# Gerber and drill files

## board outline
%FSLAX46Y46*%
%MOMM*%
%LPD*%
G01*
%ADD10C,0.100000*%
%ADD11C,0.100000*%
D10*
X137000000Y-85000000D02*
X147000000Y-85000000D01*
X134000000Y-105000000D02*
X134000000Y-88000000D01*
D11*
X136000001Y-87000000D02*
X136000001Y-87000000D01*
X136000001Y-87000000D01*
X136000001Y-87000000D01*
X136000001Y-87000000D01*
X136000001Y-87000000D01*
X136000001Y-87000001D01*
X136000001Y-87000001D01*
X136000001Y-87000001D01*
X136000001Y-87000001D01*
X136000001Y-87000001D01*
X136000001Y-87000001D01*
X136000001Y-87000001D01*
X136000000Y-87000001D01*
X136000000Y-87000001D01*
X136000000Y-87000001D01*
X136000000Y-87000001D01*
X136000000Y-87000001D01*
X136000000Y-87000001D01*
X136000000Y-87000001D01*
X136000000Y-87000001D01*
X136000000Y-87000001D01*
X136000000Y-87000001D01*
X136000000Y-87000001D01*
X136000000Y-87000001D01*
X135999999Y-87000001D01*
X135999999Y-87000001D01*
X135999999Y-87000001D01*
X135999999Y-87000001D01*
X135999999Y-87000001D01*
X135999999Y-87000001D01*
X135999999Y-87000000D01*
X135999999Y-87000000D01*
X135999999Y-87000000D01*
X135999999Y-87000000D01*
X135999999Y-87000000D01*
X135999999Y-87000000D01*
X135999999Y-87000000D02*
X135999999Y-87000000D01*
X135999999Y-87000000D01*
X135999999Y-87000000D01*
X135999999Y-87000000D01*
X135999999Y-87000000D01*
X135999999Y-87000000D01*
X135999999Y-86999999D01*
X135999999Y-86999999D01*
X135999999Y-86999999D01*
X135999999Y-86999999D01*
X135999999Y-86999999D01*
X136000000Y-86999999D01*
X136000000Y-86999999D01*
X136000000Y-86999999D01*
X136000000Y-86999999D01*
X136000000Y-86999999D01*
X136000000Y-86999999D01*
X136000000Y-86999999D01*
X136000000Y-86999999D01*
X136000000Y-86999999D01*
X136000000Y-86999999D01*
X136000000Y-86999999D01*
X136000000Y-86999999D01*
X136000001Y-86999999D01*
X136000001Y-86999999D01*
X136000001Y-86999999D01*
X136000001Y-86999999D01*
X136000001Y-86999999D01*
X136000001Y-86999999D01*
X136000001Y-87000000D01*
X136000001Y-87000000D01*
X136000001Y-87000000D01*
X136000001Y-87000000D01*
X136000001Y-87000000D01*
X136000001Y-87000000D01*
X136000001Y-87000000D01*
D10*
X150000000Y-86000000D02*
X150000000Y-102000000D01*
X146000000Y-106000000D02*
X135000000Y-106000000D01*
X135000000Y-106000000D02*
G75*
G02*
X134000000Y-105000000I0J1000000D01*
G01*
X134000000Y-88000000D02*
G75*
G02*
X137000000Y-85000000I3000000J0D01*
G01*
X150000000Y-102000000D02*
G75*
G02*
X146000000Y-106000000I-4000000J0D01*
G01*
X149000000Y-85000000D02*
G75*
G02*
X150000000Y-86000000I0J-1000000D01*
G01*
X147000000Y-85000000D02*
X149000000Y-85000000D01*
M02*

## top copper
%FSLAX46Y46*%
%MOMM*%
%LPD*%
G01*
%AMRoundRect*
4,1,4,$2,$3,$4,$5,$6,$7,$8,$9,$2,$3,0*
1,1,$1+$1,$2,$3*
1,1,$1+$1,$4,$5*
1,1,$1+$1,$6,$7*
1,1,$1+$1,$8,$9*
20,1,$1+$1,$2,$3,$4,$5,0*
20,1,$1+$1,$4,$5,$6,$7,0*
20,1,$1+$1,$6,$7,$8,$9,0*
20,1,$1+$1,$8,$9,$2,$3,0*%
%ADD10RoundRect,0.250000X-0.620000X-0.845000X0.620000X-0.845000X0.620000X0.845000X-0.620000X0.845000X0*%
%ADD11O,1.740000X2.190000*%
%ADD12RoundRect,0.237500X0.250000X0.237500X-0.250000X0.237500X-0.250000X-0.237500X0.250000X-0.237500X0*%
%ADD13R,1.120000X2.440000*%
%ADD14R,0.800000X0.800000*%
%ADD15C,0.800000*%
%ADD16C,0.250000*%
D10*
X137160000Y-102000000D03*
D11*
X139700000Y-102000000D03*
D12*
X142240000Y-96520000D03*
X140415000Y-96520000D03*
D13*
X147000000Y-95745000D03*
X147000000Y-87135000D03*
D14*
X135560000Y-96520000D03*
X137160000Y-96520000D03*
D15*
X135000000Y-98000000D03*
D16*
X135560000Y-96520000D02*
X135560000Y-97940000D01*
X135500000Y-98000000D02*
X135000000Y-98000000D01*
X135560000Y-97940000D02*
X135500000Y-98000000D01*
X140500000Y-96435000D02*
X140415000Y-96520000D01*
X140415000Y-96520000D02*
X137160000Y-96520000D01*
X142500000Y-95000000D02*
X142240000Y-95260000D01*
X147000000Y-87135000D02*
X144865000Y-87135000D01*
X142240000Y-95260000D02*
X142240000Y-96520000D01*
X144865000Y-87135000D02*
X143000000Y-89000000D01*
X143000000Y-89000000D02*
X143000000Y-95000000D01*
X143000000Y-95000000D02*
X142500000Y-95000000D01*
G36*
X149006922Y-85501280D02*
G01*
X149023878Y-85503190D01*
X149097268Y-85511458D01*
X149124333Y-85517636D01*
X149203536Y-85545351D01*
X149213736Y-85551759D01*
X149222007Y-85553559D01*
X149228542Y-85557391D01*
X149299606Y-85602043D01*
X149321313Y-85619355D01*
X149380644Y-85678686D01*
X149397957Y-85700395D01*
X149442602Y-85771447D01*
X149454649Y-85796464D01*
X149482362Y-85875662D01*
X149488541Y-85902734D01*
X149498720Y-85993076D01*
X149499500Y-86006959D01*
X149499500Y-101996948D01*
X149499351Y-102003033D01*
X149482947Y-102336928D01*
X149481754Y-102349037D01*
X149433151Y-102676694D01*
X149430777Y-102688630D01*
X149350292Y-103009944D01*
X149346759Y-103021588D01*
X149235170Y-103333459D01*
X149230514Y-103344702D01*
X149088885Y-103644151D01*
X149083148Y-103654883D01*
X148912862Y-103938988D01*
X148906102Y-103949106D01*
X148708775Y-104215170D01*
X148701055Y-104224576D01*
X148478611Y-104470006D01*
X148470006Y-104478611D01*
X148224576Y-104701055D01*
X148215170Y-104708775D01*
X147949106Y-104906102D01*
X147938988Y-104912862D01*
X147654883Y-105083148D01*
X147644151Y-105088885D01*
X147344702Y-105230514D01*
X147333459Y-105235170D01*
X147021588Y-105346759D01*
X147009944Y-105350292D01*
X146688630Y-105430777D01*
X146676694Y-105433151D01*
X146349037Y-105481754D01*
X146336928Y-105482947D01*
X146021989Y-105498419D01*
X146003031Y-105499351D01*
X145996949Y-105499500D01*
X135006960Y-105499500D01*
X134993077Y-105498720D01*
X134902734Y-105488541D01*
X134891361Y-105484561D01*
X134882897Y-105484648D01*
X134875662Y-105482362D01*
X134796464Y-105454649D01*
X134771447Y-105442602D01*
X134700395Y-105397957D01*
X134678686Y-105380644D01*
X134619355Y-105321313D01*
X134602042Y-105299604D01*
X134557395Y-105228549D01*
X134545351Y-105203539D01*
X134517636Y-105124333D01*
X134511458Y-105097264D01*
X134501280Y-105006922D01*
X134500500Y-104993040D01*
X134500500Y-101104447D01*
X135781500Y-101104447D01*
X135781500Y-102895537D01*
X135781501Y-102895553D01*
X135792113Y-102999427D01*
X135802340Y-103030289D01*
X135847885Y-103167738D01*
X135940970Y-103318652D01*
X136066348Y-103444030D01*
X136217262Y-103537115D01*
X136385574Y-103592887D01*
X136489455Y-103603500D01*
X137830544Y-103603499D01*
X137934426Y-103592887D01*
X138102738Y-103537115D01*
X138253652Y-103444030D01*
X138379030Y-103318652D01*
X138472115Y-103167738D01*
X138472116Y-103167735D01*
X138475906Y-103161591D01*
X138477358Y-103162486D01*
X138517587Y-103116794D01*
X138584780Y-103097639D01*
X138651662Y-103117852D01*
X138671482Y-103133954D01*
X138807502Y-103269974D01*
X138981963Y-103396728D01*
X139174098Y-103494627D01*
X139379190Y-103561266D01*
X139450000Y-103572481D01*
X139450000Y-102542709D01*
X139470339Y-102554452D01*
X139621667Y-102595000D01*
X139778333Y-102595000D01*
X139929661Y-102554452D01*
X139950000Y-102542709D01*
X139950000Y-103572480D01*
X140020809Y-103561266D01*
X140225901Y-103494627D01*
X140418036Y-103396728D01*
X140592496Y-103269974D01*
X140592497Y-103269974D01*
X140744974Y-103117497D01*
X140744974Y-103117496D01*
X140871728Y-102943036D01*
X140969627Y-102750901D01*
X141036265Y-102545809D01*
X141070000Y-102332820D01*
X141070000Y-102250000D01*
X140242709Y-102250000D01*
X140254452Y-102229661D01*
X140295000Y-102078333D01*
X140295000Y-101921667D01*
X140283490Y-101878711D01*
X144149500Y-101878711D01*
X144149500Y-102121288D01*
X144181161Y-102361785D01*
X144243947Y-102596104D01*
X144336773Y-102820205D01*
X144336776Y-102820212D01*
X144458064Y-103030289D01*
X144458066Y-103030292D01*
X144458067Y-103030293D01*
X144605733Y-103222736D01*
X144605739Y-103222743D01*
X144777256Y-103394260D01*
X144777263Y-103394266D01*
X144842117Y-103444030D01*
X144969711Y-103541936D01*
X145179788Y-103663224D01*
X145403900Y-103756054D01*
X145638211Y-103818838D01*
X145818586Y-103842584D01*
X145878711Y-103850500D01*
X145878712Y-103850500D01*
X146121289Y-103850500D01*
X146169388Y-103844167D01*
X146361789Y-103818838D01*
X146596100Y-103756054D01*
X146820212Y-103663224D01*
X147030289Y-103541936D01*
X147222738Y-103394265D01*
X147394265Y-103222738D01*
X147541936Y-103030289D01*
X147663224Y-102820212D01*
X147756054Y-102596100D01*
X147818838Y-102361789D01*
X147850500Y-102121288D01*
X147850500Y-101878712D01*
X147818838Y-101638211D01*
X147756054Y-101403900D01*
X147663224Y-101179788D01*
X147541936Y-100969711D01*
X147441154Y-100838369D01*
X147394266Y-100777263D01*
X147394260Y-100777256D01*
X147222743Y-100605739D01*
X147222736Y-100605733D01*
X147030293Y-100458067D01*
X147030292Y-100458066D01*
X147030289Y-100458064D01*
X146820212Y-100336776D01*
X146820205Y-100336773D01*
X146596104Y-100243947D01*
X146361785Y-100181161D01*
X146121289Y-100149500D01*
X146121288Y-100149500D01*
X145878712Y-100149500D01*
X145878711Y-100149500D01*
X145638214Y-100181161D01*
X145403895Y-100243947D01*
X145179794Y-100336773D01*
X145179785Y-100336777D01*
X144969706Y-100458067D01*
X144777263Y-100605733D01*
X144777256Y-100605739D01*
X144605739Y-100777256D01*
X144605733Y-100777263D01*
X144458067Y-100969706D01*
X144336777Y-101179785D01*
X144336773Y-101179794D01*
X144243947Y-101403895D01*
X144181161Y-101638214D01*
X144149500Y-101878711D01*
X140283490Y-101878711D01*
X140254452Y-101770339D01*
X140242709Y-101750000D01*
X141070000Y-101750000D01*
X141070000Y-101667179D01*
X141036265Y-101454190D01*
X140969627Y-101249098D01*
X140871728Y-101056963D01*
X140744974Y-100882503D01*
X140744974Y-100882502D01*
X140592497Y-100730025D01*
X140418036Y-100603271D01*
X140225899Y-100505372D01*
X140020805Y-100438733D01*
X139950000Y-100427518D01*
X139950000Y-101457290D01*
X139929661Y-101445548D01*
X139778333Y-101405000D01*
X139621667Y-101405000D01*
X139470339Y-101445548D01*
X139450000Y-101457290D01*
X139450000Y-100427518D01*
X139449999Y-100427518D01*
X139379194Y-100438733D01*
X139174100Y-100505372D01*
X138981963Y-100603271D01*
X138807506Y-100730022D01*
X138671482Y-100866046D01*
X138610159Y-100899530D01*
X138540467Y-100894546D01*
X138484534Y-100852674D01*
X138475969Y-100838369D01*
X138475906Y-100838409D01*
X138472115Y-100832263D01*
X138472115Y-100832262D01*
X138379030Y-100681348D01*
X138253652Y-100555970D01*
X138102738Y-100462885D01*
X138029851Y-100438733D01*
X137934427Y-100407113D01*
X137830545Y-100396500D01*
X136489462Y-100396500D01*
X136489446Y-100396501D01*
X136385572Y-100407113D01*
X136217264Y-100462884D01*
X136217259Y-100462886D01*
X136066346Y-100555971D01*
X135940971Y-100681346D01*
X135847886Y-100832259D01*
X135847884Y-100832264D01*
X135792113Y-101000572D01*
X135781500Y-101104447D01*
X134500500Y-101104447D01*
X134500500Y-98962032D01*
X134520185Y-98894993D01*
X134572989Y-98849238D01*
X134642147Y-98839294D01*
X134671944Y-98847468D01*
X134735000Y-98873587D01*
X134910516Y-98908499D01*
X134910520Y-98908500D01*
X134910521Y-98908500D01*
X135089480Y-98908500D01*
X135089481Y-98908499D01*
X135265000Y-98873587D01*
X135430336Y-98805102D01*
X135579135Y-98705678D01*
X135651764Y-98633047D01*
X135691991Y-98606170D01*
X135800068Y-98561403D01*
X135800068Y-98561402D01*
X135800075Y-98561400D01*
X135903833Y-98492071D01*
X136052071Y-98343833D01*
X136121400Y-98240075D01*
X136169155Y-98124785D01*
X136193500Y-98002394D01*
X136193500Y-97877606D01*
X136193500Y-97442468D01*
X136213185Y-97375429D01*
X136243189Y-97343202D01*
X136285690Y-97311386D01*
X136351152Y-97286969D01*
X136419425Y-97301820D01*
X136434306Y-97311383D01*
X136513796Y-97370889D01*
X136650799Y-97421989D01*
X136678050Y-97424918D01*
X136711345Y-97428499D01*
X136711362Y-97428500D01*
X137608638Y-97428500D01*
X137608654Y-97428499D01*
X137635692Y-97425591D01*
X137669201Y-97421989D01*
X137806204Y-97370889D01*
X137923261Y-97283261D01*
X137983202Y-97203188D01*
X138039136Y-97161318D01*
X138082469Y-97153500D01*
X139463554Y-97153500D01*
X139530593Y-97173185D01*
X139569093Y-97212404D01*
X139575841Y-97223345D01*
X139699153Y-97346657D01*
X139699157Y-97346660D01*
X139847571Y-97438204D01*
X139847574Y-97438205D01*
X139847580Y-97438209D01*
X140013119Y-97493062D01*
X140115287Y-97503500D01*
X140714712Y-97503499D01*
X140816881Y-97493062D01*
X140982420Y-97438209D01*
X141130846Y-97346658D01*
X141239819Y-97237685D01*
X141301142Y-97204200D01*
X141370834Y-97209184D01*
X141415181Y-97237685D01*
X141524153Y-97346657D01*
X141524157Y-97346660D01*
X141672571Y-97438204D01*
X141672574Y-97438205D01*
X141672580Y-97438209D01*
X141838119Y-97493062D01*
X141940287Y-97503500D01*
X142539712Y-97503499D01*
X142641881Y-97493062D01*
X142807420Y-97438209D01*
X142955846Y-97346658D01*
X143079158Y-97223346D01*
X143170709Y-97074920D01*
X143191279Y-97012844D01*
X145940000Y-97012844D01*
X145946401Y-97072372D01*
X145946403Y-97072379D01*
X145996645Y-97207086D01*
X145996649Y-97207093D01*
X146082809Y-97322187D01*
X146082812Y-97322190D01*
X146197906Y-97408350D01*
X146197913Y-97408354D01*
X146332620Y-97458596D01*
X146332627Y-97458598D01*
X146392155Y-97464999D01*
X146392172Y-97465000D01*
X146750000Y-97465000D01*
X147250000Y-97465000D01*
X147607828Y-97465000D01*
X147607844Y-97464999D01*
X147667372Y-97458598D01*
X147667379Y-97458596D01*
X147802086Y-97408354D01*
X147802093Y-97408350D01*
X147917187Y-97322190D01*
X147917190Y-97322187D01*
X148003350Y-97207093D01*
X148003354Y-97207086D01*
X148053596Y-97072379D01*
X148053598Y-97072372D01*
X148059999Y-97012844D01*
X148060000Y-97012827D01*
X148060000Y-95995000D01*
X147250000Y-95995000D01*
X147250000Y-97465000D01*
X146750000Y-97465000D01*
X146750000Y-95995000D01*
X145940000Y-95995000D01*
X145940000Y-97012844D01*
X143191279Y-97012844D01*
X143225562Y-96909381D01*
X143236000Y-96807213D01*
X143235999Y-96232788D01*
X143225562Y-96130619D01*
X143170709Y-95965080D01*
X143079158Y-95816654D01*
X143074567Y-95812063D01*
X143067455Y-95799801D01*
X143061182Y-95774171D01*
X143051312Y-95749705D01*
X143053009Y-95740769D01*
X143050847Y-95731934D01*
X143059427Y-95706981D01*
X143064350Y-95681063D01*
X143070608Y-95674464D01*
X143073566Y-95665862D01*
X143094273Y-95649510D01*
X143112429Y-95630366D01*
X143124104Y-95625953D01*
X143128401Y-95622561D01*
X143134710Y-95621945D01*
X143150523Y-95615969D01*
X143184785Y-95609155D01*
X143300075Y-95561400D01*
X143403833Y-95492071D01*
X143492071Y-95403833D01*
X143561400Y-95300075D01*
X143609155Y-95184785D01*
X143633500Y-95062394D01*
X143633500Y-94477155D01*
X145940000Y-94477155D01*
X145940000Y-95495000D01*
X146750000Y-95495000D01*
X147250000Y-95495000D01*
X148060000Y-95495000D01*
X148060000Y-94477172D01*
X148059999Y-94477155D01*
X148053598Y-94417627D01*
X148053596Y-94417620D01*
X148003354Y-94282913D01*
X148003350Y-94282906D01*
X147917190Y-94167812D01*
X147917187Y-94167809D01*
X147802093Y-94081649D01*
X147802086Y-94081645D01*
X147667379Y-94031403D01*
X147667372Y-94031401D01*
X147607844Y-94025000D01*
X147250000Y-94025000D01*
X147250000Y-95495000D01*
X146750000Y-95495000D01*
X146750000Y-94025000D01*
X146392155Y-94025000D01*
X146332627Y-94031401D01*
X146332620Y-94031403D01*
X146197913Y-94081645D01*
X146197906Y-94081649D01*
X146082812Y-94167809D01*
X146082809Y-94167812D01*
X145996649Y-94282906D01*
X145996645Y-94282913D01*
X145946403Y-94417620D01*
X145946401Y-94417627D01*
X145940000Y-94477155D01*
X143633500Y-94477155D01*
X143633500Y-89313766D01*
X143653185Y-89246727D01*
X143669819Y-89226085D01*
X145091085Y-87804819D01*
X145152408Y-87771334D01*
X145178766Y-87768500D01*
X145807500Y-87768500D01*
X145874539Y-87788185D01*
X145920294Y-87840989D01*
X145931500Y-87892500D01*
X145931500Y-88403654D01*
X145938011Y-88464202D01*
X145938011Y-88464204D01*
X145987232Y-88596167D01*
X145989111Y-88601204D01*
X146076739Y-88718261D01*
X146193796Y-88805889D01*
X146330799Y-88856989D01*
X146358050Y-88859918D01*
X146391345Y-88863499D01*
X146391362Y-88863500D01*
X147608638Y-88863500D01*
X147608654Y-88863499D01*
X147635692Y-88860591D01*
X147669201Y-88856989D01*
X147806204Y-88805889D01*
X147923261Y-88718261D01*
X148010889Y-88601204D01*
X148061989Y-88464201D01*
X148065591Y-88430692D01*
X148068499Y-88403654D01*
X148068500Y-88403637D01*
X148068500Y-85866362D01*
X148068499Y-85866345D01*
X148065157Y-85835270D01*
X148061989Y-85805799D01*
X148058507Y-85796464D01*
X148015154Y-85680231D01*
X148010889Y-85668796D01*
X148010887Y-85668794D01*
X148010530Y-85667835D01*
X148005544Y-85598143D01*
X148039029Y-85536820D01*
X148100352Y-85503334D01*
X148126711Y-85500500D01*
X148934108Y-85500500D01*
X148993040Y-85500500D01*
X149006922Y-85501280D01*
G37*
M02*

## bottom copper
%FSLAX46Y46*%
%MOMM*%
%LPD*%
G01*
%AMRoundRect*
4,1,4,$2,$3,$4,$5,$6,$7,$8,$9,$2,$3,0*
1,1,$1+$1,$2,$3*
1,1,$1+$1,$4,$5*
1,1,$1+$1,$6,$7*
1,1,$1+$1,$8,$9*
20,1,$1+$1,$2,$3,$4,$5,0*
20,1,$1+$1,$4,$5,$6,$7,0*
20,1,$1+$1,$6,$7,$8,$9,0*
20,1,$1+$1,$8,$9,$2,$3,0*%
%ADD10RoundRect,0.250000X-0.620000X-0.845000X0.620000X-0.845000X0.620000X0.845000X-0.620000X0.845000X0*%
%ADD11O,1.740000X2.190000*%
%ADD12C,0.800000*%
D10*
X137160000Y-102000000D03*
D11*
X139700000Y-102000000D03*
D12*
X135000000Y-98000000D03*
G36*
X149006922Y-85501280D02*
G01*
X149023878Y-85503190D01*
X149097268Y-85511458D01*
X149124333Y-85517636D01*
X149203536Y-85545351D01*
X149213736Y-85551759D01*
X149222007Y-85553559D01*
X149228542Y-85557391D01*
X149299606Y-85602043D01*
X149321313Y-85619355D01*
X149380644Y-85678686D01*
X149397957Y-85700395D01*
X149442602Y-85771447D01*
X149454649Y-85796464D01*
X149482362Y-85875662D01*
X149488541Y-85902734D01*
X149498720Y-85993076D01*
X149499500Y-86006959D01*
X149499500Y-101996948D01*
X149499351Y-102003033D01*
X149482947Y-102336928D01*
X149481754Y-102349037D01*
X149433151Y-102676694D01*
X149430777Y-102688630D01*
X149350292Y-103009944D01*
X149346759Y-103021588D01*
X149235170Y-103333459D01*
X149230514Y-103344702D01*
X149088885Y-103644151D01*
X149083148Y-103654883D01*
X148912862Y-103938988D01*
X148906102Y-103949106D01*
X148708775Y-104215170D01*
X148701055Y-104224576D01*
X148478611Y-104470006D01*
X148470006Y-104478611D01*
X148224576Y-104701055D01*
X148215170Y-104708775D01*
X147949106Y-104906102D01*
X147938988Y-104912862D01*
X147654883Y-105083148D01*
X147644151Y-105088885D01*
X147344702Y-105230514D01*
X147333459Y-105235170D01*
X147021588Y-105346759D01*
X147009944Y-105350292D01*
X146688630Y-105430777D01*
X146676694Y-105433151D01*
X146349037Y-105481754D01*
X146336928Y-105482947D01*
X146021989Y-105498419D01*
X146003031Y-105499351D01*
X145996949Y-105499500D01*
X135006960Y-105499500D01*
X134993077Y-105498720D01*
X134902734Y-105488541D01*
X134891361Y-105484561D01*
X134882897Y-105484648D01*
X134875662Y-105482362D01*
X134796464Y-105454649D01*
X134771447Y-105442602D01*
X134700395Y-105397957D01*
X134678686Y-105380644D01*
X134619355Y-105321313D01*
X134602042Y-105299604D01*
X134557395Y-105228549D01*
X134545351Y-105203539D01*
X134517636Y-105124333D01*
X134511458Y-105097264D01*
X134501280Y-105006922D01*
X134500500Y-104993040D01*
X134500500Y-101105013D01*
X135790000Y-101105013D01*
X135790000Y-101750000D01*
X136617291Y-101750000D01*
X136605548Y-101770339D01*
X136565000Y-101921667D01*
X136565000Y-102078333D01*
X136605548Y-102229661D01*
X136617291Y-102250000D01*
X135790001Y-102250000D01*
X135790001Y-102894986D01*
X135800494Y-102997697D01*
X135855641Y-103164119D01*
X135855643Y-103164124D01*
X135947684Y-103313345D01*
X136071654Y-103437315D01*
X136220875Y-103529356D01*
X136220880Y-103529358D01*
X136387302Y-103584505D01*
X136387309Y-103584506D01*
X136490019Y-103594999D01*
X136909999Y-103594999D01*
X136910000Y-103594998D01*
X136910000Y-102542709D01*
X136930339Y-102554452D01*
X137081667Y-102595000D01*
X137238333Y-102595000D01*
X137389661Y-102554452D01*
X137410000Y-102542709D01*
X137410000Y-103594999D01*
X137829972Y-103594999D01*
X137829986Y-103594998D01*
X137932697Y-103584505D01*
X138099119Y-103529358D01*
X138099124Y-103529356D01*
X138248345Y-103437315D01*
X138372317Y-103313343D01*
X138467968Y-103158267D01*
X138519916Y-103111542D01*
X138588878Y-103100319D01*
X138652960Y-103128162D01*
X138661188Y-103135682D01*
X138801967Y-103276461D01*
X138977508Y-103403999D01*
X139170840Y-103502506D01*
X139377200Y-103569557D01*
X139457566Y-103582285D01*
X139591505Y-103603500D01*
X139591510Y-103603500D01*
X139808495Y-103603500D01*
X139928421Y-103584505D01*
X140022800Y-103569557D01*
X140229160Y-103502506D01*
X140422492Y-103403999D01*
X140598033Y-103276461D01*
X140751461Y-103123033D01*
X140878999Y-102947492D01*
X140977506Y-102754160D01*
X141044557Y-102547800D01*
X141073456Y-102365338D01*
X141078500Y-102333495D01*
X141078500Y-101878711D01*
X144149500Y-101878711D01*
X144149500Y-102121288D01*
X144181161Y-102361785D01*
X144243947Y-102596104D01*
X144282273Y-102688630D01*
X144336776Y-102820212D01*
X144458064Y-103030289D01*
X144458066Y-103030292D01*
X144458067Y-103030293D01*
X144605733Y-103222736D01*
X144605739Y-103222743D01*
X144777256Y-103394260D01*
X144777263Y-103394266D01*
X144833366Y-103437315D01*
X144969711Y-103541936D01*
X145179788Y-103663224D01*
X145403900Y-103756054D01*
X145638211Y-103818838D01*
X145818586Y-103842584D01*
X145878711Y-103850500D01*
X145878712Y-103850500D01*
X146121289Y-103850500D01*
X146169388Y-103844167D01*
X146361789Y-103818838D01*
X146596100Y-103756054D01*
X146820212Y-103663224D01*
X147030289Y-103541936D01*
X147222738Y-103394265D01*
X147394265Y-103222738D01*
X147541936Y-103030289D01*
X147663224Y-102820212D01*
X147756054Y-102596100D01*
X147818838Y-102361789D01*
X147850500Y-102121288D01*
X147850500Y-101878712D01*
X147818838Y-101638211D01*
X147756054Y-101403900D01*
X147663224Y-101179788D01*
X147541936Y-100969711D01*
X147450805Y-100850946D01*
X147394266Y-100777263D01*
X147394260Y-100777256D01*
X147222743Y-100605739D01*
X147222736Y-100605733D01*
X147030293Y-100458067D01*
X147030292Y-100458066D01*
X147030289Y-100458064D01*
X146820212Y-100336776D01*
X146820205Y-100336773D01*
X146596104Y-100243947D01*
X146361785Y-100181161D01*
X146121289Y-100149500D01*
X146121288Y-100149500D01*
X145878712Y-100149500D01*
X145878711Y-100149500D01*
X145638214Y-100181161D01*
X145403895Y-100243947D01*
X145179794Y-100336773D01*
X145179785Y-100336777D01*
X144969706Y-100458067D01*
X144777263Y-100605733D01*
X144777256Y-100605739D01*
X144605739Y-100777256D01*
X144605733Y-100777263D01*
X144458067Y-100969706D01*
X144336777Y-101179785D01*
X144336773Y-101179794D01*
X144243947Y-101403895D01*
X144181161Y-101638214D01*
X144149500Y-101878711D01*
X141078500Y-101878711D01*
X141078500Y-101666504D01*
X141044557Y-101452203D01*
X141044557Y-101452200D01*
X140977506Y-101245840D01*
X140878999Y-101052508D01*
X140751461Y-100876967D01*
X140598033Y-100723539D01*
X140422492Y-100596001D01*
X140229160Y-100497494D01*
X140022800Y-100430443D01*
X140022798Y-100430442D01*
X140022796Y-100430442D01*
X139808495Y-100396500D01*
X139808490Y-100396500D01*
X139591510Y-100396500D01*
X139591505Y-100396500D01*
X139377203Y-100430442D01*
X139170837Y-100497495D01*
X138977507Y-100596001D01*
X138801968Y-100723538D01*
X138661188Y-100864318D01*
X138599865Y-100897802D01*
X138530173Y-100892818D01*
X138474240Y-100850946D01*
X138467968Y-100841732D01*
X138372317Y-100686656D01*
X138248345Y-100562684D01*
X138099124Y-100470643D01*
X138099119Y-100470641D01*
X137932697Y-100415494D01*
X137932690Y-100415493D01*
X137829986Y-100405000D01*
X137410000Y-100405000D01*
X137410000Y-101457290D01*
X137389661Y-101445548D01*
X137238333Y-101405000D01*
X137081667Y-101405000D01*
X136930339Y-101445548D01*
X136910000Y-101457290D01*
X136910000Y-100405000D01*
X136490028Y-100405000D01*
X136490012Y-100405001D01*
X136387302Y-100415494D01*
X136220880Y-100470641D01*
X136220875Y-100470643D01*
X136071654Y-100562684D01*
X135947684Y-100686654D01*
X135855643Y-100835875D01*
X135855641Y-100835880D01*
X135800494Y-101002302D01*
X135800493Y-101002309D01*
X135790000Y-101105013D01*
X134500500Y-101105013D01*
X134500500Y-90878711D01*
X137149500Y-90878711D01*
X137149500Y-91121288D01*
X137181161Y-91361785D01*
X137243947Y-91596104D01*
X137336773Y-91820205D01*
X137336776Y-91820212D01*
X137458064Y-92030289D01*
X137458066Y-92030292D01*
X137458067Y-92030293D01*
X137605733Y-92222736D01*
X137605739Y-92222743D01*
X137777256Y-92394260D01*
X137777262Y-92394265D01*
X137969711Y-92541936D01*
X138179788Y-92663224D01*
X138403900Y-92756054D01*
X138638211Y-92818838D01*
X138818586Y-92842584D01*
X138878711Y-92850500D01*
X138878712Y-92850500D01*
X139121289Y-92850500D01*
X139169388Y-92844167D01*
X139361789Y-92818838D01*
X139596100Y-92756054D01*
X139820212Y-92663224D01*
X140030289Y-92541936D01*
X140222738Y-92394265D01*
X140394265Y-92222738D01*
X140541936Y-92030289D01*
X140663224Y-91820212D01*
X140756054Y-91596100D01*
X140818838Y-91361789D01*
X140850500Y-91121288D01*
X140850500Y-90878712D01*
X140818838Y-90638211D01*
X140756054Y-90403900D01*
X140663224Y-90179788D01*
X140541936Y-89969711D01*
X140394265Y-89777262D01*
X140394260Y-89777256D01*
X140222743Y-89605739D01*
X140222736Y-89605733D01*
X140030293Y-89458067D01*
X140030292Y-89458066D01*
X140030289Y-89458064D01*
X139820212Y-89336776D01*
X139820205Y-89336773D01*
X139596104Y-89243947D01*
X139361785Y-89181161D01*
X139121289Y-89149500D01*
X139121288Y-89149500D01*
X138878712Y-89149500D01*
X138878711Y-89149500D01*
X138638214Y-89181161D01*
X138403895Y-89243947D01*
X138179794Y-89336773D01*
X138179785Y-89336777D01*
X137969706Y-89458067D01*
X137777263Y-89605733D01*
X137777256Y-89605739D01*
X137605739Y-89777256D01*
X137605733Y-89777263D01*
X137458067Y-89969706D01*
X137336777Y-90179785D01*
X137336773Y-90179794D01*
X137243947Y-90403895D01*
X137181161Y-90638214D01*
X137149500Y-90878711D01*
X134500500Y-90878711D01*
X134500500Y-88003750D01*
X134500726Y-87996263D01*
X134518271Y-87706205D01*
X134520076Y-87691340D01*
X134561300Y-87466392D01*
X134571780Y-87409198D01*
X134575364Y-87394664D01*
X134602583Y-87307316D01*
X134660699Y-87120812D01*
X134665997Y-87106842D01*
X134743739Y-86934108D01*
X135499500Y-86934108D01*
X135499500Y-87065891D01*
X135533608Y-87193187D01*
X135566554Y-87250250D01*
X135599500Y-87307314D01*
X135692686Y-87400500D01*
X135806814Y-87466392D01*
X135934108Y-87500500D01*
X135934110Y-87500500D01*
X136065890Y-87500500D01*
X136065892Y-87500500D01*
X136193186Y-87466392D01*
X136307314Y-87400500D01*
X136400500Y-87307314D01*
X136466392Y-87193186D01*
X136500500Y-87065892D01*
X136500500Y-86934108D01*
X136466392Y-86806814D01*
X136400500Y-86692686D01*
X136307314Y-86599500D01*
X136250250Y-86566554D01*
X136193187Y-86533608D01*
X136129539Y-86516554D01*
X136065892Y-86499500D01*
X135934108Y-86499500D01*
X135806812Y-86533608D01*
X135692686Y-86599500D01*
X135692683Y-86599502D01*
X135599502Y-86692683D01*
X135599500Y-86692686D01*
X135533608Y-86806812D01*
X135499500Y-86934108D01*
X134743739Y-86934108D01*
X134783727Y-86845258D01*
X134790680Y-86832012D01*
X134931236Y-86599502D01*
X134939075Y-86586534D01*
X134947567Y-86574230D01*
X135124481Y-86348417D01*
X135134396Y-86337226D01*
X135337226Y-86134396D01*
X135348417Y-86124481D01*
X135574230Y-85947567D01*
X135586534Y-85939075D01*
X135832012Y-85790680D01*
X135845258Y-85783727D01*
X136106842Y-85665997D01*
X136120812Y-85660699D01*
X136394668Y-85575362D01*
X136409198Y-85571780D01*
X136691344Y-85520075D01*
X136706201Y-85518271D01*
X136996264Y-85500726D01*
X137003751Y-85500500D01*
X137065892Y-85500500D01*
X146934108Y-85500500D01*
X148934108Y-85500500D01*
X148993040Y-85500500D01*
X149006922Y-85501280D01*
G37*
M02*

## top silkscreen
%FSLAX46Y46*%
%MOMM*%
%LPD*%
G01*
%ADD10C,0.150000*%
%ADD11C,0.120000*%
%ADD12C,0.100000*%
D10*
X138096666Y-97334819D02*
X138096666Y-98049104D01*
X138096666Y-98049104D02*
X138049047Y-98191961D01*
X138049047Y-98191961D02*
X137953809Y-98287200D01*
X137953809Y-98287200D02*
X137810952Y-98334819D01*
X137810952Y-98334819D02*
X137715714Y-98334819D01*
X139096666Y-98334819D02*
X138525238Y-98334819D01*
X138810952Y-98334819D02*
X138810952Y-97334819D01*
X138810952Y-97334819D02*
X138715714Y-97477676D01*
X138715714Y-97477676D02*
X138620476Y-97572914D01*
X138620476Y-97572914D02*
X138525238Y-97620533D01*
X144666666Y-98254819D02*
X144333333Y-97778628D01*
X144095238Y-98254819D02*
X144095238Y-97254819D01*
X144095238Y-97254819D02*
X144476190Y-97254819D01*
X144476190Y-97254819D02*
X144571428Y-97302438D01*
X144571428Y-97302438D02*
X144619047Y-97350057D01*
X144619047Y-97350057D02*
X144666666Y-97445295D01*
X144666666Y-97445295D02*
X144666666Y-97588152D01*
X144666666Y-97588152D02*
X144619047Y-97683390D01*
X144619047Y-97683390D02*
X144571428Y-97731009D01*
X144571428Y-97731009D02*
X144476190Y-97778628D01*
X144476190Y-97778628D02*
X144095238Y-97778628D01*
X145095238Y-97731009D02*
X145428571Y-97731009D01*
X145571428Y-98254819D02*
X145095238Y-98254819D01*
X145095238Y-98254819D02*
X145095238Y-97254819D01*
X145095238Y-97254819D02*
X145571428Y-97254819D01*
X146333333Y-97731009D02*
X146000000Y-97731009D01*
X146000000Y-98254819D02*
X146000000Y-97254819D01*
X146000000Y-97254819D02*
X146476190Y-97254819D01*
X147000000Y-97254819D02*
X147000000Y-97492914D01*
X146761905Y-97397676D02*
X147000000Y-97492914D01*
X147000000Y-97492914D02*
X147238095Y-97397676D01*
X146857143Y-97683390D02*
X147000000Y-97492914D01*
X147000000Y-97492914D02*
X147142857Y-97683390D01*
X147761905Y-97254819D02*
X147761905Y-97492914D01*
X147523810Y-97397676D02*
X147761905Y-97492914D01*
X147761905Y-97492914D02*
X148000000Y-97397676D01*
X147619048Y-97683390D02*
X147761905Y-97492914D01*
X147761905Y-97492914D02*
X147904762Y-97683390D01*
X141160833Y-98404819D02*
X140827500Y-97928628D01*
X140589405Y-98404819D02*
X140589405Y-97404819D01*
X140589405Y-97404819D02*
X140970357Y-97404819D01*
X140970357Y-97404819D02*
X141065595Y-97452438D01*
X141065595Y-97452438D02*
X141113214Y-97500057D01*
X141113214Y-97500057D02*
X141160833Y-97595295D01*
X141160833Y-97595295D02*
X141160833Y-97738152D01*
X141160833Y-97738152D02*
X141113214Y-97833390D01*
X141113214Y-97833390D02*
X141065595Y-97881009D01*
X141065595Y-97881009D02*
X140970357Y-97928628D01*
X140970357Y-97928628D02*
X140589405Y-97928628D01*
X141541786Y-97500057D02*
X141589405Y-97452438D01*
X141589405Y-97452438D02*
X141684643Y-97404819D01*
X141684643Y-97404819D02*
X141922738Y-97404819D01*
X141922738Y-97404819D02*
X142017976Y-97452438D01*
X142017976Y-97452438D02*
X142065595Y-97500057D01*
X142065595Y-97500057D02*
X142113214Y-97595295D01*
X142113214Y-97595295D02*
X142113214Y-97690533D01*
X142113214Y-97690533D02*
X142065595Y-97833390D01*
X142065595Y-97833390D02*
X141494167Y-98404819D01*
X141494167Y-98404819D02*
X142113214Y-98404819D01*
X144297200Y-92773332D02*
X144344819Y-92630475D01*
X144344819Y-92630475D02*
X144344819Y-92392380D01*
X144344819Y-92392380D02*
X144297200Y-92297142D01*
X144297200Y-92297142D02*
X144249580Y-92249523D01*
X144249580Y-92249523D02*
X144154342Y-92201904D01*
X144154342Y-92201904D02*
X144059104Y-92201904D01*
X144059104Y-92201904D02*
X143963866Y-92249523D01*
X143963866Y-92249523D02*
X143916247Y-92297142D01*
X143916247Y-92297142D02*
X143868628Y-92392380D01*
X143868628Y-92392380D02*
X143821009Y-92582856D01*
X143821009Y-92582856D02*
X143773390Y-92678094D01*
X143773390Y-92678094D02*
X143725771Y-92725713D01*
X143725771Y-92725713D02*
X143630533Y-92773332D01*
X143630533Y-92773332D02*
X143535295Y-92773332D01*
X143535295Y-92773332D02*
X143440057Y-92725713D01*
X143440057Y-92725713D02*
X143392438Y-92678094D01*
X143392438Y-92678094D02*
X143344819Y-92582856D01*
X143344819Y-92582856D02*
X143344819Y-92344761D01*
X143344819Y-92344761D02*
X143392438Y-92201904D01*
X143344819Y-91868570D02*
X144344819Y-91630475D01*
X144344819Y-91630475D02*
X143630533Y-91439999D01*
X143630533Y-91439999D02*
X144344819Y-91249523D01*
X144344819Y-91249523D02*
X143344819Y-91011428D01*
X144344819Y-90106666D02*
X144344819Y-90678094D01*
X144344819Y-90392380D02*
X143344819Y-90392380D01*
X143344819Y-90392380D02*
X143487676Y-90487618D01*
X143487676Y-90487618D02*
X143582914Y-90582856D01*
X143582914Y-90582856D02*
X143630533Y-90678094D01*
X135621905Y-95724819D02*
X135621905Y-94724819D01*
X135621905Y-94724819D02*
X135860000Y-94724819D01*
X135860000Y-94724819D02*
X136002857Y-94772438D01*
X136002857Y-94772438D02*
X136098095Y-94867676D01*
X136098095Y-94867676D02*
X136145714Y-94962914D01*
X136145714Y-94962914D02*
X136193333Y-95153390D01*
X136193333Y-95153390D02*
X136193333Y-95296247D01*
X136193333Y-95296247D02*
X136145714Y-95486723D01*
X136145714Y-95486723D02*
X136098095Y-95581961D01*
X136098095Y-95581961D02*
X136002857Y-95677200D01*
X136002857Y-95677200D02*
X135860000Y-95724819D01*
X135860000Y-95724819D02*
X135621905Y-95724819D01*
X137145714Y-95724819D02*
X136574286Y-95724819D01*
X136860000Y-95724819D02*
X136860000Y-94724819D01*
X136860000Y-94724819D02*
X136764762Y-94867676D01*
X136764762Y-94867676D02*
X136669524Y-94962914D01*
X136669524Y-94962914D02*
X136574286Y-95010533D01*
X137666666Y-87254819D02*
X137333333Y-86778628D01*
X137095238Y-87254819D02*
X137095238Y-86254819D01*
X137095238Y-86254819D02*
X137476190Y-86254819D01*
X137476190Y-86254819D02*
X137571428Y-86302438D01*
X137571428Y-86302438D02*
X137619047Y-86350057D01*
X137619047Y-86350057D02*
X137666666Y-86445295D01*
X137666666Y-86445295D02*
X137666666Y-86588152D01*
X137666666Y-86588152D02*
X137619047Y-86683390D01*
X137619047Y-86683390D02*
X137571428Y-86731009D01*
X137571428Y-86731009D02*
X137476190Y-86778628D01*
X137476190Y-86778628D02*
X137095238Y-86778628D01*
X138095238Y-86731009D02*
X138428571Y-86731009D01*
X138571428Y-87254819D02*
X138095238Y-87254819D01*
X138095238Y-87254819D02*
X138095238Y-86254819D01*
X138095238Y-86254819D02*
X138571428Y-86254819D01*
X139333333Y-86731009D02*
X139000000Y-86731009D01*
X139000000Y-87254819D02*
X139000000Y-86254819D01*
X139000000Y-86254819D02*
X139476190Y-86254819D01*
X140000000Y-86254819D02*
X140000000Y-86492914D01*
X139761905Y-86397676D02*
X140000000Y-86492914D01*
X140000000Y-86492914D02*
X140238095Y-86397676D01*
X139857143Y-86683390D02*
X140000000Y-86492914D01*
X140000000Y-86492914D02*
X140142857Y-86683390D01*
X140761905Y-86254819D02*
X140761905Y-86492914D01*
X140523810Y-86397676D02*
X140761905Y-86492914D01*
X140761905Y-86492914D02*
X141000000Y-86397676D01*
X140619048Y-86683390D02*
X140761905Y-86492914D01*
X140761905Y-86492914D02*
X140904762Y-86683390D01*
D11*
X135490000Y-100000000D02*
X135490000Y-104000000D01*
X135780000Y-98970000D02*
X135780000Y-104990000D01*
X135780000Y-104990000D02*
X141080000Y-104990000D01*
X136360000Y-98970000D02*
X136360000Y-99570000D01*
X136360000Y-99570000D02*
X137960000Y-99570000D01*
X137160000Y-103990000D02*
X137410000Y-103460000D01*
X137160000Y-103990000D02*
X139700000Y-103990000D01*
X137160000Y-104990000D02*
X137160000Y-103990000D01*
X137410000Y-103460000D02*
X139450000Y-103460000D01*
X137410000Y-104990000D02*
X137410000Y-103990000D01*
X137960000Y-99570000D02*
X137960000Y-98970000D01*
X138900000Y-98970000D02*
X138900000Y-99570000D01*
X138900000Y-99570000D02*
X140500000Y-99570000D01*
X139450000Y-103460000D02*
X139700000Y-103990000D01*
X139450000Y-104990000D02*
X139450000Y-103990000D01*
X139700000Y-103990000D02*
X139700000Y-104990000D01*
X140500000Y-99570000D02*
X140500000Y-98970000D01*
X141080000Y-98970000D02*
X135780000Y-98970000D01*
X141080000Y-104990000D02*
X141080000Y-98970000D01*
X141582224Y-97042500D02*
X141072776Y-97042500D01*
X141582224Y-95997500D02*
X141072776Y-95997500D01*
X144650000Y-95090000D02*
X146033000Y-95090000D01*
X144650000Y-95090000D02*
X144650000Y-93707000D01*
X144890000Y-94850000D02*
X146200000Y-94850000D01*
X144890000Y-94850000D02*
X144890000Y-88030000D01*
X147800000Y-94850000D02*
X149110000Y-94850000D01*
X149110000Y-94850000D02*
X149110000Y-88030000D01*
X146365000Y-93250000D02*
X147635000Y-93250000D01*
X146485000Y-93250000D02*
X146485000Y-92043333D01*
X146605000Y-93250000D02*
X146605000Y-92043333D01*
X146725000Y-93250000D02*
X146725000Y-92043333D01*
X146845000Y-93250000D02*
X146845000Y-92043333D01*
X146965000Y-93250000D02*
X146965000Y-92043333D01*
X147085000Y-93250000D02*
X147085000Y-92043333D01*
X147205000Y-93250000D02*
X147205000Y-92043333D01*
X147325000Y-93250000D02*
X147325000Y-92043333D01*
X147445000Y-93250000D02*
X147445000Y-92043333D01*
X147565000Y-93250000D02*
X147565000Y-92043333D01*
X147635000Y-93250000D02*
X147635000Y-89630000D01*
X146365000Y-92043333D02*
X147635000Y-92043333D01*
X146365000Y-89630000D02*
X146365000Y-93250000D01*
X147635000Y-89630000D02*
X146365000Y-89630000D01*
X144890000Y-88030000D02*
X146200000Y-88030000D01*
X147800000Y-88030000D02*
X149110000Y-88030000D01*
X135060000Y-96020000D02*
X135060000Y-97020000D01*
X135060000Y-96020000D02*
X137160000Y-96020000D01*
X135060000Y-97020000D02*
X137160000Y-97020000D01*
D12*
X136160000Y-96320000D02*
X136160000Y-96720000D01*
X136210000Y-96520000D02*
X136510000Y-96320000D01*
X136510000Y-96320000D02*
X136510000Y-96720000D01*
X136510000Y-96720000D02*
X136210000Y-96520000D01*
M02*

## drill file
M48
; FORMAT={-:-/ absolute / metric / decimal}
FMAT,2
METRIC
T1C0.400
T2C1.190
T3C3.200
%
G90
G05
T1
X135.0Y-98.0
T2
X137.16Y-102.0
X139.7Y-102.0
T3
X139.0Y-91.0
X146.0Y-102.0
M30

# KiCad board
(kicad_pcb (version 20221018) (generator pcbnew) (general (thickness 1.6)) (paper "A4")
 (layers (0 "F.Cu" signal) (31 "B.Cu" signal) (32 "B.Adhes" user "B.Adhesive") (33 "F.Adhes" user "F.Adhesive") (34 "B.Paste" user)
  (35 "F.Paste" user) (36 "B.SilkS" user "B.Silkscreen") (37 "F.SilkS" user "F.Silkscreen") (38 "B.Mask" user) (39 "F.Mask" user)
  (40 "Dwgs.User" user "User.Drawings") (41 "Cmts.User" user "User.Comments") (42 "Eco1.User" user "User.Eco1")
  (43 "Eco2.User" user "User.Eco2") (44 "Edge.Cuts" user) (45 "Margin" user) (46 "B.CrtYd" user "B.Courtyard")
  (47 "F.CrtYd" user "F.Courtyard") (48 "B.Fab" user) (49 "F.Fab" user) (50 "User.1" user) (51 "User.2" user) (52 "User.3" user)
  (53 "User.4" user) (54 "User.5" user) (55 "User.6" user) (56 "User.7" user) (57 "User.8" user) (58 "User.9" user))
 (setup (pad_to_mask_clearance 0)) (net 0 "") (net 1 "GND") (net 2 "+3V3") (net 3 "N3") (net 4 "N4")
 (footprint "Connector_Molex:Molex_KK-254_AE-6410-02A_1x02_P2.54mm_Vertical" (layer "F.Cu") (at 137.16 102)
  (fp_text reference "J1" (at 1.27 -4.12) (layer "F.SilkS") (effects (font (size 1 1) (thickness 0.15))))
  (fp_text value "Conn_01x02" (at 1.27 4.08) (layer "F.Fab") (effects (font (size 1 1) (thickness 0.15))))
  (fp_line (start -1.67 -2) (end -1.67 2) (stroke (width 0.12) (type solid)) (layer "F.SilkS"))
  (fp_line (start -1.38 -3.03) (end -1.38 2.99) (stroke (width 0.12) (type solid)) (layer "F.SilkS"))
  (fp_line (start -1.38 2.99) (end 3.92 2.99) (stroke (width 0.12) (type solid)) (layer "F.SilkS"))
  (fp_line (start -0.8 -3.03) (end -0.8 -2.43) (stroke (width 0.12) (type solid)) (layer "F.SilkS"))
  (fp_line (start -0.8 -2.43) (end 0.8 -2.43) (stroke (width 0.12) (type solid)) (layer "F.SilkS"))
  (fp_line (start 0 1.99) (end 0.25 1.46) (stroke (width 0.12) (type solid)) (layer "F.SilkS"))
  (fp_line (start 0 1.99) (end 2.54 1.99) (stroke (width 0.12) (type solid)) (layer "F.SilkS"))
  (fp_line (start 0 2.99) (end 0 1.99) (stroke (width 0.12) (type solid)) (layer "F.SilkS"))
  (fp_line (start 0.25 1.46) (end 2.29 1.46) (stroke (width 0.12) (type solid)) (layer "F.SilkS"))
  (fp_line (start 0.25 2.99) (end 0.25 1.99) (stroke (width 0.12) (type solid)) (layer "F.SilkS"))
  (fp_line (start 0.8 -2.43) (end 0.8 -3.03) (stroke (width 0.12) (type solid)) (layer "F.SilkS"))
  (fp_line (start 1.74 -3.03) (end 1.74 -2.43) (stroke (width 0.12) (type solid)) (layer "F.SilkS"))
  (fp_line (start 1.74 -2.43) (end 3.34 -2.43) (stroke (width 0.12) (type solid)) (layer "F.SilkS"))
  (fp_line (start 2.29 1.46) (end 2.54 1.99) (stroke (width 0.12) (type solid)) (layer "F.SilkS"))
  (fp_line (start 2.29 2.99) (end 2.29 1.99) (stroke (width 0.12) (type solid)) (layer "F.SilkS"))
  (fp_line (start 2.54 1.99) (end 2.54 2.99) (stroke (width 0.12) (type solid)) (layer "F.SilkS"))
  (fp_line (start 3.34 -2.43) (end 3.34 -3.03) (stroke (width 0.12) (type solid)) (layer "F.SilkS"))
  (fp_line (start 3.92 -3.03) (end -1.38 -3.03) (stroke (width 0.12) (type solid)) (layer "F.SilkS"))
  (fp_line (start 3.92 2.99) (end 3.92 -3.03) (stroke (width 0.12) (type solid)) (layer "F.SilkS"))
  (pad "1" thru_hole roundrect (at 0 0) (size 1.74 2.19) (drill 1.19) (layers "*.Cu" "*.Mask") (roundrect_rratio 0.143678) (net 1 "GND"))
  (pad "2" thru_hole oval (at 2.54 0) (size 1.74 2.19) (drill 1.19) (layers "*.Cu" "*.Mask") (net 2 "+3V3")))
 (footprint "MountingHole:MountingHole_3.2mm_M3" (layer "F.Cu") (at 146 102)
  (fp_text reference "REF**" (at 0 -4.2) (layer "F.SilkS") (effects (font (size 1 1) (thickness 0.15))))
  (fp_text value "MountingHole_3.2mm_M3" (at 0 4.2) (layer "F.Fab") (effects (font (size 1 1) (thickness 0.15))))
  (pad "" np_thru_hole circle (at 0 0) (size 3.2 3.2) (drill 3.2) (layers "*.Cu" "*.Mask")))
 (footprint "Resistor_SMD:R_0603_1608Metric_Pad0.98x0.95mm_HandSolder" (layer "F.Cu") (at 141.3275 96.52 180)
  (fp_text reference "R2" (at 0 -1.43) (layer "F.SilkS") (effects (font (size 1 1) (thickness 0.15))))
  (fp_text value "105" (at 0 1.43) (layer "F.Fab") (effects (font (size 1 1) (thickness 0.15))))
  (fp_line (start -0.254724 -0.5225) (end 0.254724 -0.5225) (stroke (width 0.12) (type solid)) (layer "F.SilkS"))
  (fp_line (start -0.254724 0.5225) (end 0.254724 0.5225) (stroke (width 0.12) (type solid)) (layer "F.SilkS"))
  (pad "1" smd roundrect (at -0.9125 0 180) (size 0.975 0.95) (layers "F.Cu" "F.Paste" "F.Mask") (roundrect_rratio 0.25) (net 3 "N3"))
  (pad "2" smd roundrect (at 0.9125 0 180) (size 0.975 0.95) (layers "F.Cu" "F.Paste" "F.Mask") (roundrect_rratio 0.25) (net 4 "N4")))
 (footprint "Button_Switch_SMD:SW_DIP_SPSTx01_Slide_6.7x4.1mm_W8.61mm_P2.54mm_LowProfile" (layer "F.Cu") (at 147 91.44 90)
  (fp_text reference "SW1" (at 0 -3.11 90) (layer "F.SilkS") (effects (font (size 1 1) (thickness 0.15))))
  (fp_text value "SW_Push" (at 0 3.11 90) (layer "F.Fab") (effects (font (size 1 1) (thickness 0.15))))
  (fp_line (start -3.65 -2.35) (end -3.65 -0.967) (stroke (width 0.12) (type solid)) (layer "F.SilkS"))
  (fp_line (start -3.65 -2.35) (end -2.267 -2.35) (stroke (width 0.12) (type solid)) (layer "F.SilkS"))
  (fp_line (start -3.41 -2.11) (end -3.41 -0.8) (stroke (width 0.12) (type solid)) (layer "F.SilkS"))
  (fp_line (start -3.41 -2.11) (end 3.41 -2.11) (stroke (width 0.12) (type solid)) (layer "F.SilkS"))
  (fp_line (start -3.41 0.8) (end -3.41 2.11) (stroke (width 0.12) (type solid)) (layer "F.SilkS"))
  (fp_line (start -3.41 2.11) (end 3.41 2.11) (stroke (width 0.12) (type solid)) (layer "F.SilkS"))
  (fp_line (start -1.81 -0.635) (end -1.81 0.635) (stroke (width 0.12) (type solid)) (layer "F.SilkS"))
  (fp_line (start -1.81 -0.515) (end -0.603333 -0.515) (stroke (width 0.12) (type solid)) (layer "F.SilkS"))
  (fp_line (start -1.81 -0.395) (end -0.603333 -0.395) (stroke (width 0.12) (type solid)) (layer "F.SilkS"))
  (fp_line (start -1.81 -0.275) (end -0.603333 -0.275) (stroke (width 0.12) (type solid)) (layer "F.SilkS"))
  (fp_line (start -1.81 -0.155) (end -0.603333 -0.155) (stroke (width 0.12) (type solid)) (layer "F.SilkS"))
  (fp_line (start -1.81 -0.035) (end -0.603333 -0.035) (stroke (width 0.12) (type solid)) (layer "F.SilkS"))
  (fp_line (start -1.81 0.085) (end -0.603333 0.085) (stroke (width 0.12) (type solid)) (layer "F.SilkS"))
  (fp_line (start -1.81 0.205) (end -0.603333 0.205) (stroke (width 0.12) (type solid)) (layer "F.SilkS"))
  (fp_line (start -1.81 0.325) (end -0.603333 0.325) (stroke (width 0.12) (type solid)) (layer "F.SilkS"))
  (fp_line (start -1.81 0.445) (end -0.603333 0.445) (stroke (width 0.12) (type solid)) (layer "F.SilkS"))
  (fp_line (start -1.81 0.565) (end -0.603333 0.565) (stroke (width 0.12) (type solid)) (layer "F.SilkS"))
  (fp_line (start -1.81 0.635) (end 1.81 0.635) (stroke (width 0.12) (type solid)) (layer "F.SilkS"))
  (fp_line (start -0.603333 -0.635) (end -0.603333 0.635) (stroke (width 0.12) (type solid)) (layer "F.SilkS"))
  (fp_line (start 1.81 -0.635) (end -1.81 -0.635) (stroke (width 0.12) (type solid)) (layer "F.SilkS"))
  (fp_line (start 1.81 0.635) (end 1.81 -0.635) (stroke (width 0.12) (type solid)) (layer "F.SilkS"))
  (fp_line (start 3.41 -2.11) (end 3.41 -0.8) (stroke (width 0.12) (type solid)) (layer "F.SilkS"))
  (fp_line (start 3.41 0.8) (end 3.41 2.11) (stroke (width 0.12) (type solid)) (layer "F.SilkS"))
  (pad "1" smd rect (at -4.305 0 90) (size 2.44 1.12) (layers "F.Cu" "F.Paste" "F.Mask") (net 2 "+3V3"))
  (pad "2" smd rect (at 4.305 0 90) (size 2.44 1.12) (layers "F.Cu" "F.Paste" "F.Mask") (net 3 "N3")))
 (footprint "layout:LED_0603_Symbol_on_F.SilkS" (layer "F.Cu") (at 136.36 96.52)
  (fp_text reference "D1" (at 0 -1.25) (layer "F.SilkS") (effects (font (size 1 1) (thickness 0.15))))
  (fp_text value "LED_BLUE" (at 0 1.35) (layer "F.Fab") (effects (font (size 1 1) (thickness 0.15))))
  (fp_line (start -1.3 -0.5) (end -1.3 0.5) (stroke (width 0.12) (type solid)) (layer "F.SilkS"))
  (fp_line (start -1.3 -0.5) (end 0.8 -0.5) (stroke (width 0.12) (type solid)) (layer "F.SilkS"))
  (fp_line (start -1.3 0.5) (end 0.8 0.5) (stroke (width 0.12) (type solid)) (layer "F.SilkS"))
  (fp_line (start -0.2 -0.2) (end -0.2 0.2) (stroke (width 0.1) (type solid)) (layer "F.SilkS"))
  (fp_line (start -0.15 0) (end 0.15 -0.2) (stroke (width 0.1) (type solid)) (layer "F.SilkS"))
  (fp_line (start 0.15 -0.2) (end 0.15 0.2) (stroke (width 0.1) (type solid)) (layer "F.SilkS"))
  (fp_line (start 0.15 0.2) (end -0.15 0) (stroke (width 0.1) (type solid)) (layer "F.SilkS"))
  (pad "1" smd rect (at -0.8 0 180) (size 0.8 0.8) (layers "F.Cu" "F.Paste" "F.Mask") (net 1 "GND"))
  (pad "2" smd rect (at 0.8 0 180) (size 0.8 0.8) (layers "F.Cu" "F.Paste" "F.Mask") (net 4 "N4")))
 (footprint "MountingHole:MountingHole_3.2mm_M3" (layer "F.Cu") (at 139 91)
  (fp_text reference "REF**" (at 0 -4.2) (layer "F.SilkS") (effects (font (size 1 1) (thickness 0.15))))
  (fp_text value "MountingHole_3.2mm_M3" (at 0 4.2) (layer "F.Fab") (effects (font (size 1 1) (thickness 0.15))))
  (pad "" np_thru_hole circle (at 0 0) (size 3.2 3.2) (drill 3.2) (layers "*.Cu" "*.Mask")))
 (gr_line (start 137 85) (end 147 85) (stroke (width 0.1) (type default)) (layer "Edge.Cuts"))
 (gr_line (start 134 105) (end 134 88) (stroke (width 0.1) (type default)) (layer "Edge.Cuts"))
 (gr_arc (start 136 87) (mid 136 87) (end 136 87) (stroke (width 0.1) (type default)) (layer "Edge.Cuts"))
 (gr_line (start 150 86) (end 150 102) (stroke (width 0.1) (type default)) (layer "Edge.Cuts"))
 (gr_line (start 146 106) (end 135 106) (stroke (width 0.1) (type default)) (layer "Edge.Cuts"))
 (gr_arc (start 135 106) (mid 134.292893 105.707107) (end 134 105) (stroke (width 0.1) (type default)) (layer "Edge.Cuts"))
 (gr_arc (start 134 88) (mid 134.87868 85.87868) (end 137 85) (stroke (width 0.1) (type default)) (layer "Edge.Cuts"))
 (gr_arc (start 150 102) (mid 148.828427 104.828427) (end 146 106) (stroke (width 0.1) (type default)) (layer "Edge.Cuts"))
 (gr_arc (start 149 85) (mid 149.707107 85.292893) (end 150 86) (stroke (width 0.1) (type default)) (layer "Edge.Cuts"))
 (gr_line (start 147 85) (end 149 85) (stroke (width 0.1) (type default)) (layer "Edge.Cuts"))
 (segment (start 135.56 96.52) (end 135.56 97.94) (width 0.25) (layer "F.Cu") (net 1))
 (segment (start 135.5 98) (end 135 98) (width 0.25) (layer "F.Cu") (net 1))
 (segment (start 135.56 97.94) (end 135.5 98) (width 0.25) (layer "F.Cu") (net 1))
 (via (at 135 98) (size 0.8) (drill 0.4) (layers "F.Cu" "B.Cu") (free) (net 1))
 (segment (start 140.5 96.435) (end 140.415 96.52) (width 0.25) (layer "F.Cu") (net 4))
 (segment (start 140.415 96.52) (end 137.16 96.52) (width 0.25) (layer "F.Cu") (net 4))
 (segment (start 142.5 95) (end 142.24 95.26) (width 0.25) (layer "F.Cu") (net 3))
 (segment (start 147 87.135) (end 144.865 87.135) (width 0.25) (layer "F.Cu") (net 3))
 (segment (start 142.24 95.26) (end 142.24 96.52) (width 0.25) (layer "F.Cu") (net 3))
 (segment (start 144.865 87.135) (end 143 89) (width 0.25) (layer "F.Cu") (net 3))
 (segment (start 143 89) (end 143 95) (width 0.25) (layer "F.Cu") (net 3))
 (segment (start 143 95) (end 142.5 95) (width 0.25) (layer "F.Cu") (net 3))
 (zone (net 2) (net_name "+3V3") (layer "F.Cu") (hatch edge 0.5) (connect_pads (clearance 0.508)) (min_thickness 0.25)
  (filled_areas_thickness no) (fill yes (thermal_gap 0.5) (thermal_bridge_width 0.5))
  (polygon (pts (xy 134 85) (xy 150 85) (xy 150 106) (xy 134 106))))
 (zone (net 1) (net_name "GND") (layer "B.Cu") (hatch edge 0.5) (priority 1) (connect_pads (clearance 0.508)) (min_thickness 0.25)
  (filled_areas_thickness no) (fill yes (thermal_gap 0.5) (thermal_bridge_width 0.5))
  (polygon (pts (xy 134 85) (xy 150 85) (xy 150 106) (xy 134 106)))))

